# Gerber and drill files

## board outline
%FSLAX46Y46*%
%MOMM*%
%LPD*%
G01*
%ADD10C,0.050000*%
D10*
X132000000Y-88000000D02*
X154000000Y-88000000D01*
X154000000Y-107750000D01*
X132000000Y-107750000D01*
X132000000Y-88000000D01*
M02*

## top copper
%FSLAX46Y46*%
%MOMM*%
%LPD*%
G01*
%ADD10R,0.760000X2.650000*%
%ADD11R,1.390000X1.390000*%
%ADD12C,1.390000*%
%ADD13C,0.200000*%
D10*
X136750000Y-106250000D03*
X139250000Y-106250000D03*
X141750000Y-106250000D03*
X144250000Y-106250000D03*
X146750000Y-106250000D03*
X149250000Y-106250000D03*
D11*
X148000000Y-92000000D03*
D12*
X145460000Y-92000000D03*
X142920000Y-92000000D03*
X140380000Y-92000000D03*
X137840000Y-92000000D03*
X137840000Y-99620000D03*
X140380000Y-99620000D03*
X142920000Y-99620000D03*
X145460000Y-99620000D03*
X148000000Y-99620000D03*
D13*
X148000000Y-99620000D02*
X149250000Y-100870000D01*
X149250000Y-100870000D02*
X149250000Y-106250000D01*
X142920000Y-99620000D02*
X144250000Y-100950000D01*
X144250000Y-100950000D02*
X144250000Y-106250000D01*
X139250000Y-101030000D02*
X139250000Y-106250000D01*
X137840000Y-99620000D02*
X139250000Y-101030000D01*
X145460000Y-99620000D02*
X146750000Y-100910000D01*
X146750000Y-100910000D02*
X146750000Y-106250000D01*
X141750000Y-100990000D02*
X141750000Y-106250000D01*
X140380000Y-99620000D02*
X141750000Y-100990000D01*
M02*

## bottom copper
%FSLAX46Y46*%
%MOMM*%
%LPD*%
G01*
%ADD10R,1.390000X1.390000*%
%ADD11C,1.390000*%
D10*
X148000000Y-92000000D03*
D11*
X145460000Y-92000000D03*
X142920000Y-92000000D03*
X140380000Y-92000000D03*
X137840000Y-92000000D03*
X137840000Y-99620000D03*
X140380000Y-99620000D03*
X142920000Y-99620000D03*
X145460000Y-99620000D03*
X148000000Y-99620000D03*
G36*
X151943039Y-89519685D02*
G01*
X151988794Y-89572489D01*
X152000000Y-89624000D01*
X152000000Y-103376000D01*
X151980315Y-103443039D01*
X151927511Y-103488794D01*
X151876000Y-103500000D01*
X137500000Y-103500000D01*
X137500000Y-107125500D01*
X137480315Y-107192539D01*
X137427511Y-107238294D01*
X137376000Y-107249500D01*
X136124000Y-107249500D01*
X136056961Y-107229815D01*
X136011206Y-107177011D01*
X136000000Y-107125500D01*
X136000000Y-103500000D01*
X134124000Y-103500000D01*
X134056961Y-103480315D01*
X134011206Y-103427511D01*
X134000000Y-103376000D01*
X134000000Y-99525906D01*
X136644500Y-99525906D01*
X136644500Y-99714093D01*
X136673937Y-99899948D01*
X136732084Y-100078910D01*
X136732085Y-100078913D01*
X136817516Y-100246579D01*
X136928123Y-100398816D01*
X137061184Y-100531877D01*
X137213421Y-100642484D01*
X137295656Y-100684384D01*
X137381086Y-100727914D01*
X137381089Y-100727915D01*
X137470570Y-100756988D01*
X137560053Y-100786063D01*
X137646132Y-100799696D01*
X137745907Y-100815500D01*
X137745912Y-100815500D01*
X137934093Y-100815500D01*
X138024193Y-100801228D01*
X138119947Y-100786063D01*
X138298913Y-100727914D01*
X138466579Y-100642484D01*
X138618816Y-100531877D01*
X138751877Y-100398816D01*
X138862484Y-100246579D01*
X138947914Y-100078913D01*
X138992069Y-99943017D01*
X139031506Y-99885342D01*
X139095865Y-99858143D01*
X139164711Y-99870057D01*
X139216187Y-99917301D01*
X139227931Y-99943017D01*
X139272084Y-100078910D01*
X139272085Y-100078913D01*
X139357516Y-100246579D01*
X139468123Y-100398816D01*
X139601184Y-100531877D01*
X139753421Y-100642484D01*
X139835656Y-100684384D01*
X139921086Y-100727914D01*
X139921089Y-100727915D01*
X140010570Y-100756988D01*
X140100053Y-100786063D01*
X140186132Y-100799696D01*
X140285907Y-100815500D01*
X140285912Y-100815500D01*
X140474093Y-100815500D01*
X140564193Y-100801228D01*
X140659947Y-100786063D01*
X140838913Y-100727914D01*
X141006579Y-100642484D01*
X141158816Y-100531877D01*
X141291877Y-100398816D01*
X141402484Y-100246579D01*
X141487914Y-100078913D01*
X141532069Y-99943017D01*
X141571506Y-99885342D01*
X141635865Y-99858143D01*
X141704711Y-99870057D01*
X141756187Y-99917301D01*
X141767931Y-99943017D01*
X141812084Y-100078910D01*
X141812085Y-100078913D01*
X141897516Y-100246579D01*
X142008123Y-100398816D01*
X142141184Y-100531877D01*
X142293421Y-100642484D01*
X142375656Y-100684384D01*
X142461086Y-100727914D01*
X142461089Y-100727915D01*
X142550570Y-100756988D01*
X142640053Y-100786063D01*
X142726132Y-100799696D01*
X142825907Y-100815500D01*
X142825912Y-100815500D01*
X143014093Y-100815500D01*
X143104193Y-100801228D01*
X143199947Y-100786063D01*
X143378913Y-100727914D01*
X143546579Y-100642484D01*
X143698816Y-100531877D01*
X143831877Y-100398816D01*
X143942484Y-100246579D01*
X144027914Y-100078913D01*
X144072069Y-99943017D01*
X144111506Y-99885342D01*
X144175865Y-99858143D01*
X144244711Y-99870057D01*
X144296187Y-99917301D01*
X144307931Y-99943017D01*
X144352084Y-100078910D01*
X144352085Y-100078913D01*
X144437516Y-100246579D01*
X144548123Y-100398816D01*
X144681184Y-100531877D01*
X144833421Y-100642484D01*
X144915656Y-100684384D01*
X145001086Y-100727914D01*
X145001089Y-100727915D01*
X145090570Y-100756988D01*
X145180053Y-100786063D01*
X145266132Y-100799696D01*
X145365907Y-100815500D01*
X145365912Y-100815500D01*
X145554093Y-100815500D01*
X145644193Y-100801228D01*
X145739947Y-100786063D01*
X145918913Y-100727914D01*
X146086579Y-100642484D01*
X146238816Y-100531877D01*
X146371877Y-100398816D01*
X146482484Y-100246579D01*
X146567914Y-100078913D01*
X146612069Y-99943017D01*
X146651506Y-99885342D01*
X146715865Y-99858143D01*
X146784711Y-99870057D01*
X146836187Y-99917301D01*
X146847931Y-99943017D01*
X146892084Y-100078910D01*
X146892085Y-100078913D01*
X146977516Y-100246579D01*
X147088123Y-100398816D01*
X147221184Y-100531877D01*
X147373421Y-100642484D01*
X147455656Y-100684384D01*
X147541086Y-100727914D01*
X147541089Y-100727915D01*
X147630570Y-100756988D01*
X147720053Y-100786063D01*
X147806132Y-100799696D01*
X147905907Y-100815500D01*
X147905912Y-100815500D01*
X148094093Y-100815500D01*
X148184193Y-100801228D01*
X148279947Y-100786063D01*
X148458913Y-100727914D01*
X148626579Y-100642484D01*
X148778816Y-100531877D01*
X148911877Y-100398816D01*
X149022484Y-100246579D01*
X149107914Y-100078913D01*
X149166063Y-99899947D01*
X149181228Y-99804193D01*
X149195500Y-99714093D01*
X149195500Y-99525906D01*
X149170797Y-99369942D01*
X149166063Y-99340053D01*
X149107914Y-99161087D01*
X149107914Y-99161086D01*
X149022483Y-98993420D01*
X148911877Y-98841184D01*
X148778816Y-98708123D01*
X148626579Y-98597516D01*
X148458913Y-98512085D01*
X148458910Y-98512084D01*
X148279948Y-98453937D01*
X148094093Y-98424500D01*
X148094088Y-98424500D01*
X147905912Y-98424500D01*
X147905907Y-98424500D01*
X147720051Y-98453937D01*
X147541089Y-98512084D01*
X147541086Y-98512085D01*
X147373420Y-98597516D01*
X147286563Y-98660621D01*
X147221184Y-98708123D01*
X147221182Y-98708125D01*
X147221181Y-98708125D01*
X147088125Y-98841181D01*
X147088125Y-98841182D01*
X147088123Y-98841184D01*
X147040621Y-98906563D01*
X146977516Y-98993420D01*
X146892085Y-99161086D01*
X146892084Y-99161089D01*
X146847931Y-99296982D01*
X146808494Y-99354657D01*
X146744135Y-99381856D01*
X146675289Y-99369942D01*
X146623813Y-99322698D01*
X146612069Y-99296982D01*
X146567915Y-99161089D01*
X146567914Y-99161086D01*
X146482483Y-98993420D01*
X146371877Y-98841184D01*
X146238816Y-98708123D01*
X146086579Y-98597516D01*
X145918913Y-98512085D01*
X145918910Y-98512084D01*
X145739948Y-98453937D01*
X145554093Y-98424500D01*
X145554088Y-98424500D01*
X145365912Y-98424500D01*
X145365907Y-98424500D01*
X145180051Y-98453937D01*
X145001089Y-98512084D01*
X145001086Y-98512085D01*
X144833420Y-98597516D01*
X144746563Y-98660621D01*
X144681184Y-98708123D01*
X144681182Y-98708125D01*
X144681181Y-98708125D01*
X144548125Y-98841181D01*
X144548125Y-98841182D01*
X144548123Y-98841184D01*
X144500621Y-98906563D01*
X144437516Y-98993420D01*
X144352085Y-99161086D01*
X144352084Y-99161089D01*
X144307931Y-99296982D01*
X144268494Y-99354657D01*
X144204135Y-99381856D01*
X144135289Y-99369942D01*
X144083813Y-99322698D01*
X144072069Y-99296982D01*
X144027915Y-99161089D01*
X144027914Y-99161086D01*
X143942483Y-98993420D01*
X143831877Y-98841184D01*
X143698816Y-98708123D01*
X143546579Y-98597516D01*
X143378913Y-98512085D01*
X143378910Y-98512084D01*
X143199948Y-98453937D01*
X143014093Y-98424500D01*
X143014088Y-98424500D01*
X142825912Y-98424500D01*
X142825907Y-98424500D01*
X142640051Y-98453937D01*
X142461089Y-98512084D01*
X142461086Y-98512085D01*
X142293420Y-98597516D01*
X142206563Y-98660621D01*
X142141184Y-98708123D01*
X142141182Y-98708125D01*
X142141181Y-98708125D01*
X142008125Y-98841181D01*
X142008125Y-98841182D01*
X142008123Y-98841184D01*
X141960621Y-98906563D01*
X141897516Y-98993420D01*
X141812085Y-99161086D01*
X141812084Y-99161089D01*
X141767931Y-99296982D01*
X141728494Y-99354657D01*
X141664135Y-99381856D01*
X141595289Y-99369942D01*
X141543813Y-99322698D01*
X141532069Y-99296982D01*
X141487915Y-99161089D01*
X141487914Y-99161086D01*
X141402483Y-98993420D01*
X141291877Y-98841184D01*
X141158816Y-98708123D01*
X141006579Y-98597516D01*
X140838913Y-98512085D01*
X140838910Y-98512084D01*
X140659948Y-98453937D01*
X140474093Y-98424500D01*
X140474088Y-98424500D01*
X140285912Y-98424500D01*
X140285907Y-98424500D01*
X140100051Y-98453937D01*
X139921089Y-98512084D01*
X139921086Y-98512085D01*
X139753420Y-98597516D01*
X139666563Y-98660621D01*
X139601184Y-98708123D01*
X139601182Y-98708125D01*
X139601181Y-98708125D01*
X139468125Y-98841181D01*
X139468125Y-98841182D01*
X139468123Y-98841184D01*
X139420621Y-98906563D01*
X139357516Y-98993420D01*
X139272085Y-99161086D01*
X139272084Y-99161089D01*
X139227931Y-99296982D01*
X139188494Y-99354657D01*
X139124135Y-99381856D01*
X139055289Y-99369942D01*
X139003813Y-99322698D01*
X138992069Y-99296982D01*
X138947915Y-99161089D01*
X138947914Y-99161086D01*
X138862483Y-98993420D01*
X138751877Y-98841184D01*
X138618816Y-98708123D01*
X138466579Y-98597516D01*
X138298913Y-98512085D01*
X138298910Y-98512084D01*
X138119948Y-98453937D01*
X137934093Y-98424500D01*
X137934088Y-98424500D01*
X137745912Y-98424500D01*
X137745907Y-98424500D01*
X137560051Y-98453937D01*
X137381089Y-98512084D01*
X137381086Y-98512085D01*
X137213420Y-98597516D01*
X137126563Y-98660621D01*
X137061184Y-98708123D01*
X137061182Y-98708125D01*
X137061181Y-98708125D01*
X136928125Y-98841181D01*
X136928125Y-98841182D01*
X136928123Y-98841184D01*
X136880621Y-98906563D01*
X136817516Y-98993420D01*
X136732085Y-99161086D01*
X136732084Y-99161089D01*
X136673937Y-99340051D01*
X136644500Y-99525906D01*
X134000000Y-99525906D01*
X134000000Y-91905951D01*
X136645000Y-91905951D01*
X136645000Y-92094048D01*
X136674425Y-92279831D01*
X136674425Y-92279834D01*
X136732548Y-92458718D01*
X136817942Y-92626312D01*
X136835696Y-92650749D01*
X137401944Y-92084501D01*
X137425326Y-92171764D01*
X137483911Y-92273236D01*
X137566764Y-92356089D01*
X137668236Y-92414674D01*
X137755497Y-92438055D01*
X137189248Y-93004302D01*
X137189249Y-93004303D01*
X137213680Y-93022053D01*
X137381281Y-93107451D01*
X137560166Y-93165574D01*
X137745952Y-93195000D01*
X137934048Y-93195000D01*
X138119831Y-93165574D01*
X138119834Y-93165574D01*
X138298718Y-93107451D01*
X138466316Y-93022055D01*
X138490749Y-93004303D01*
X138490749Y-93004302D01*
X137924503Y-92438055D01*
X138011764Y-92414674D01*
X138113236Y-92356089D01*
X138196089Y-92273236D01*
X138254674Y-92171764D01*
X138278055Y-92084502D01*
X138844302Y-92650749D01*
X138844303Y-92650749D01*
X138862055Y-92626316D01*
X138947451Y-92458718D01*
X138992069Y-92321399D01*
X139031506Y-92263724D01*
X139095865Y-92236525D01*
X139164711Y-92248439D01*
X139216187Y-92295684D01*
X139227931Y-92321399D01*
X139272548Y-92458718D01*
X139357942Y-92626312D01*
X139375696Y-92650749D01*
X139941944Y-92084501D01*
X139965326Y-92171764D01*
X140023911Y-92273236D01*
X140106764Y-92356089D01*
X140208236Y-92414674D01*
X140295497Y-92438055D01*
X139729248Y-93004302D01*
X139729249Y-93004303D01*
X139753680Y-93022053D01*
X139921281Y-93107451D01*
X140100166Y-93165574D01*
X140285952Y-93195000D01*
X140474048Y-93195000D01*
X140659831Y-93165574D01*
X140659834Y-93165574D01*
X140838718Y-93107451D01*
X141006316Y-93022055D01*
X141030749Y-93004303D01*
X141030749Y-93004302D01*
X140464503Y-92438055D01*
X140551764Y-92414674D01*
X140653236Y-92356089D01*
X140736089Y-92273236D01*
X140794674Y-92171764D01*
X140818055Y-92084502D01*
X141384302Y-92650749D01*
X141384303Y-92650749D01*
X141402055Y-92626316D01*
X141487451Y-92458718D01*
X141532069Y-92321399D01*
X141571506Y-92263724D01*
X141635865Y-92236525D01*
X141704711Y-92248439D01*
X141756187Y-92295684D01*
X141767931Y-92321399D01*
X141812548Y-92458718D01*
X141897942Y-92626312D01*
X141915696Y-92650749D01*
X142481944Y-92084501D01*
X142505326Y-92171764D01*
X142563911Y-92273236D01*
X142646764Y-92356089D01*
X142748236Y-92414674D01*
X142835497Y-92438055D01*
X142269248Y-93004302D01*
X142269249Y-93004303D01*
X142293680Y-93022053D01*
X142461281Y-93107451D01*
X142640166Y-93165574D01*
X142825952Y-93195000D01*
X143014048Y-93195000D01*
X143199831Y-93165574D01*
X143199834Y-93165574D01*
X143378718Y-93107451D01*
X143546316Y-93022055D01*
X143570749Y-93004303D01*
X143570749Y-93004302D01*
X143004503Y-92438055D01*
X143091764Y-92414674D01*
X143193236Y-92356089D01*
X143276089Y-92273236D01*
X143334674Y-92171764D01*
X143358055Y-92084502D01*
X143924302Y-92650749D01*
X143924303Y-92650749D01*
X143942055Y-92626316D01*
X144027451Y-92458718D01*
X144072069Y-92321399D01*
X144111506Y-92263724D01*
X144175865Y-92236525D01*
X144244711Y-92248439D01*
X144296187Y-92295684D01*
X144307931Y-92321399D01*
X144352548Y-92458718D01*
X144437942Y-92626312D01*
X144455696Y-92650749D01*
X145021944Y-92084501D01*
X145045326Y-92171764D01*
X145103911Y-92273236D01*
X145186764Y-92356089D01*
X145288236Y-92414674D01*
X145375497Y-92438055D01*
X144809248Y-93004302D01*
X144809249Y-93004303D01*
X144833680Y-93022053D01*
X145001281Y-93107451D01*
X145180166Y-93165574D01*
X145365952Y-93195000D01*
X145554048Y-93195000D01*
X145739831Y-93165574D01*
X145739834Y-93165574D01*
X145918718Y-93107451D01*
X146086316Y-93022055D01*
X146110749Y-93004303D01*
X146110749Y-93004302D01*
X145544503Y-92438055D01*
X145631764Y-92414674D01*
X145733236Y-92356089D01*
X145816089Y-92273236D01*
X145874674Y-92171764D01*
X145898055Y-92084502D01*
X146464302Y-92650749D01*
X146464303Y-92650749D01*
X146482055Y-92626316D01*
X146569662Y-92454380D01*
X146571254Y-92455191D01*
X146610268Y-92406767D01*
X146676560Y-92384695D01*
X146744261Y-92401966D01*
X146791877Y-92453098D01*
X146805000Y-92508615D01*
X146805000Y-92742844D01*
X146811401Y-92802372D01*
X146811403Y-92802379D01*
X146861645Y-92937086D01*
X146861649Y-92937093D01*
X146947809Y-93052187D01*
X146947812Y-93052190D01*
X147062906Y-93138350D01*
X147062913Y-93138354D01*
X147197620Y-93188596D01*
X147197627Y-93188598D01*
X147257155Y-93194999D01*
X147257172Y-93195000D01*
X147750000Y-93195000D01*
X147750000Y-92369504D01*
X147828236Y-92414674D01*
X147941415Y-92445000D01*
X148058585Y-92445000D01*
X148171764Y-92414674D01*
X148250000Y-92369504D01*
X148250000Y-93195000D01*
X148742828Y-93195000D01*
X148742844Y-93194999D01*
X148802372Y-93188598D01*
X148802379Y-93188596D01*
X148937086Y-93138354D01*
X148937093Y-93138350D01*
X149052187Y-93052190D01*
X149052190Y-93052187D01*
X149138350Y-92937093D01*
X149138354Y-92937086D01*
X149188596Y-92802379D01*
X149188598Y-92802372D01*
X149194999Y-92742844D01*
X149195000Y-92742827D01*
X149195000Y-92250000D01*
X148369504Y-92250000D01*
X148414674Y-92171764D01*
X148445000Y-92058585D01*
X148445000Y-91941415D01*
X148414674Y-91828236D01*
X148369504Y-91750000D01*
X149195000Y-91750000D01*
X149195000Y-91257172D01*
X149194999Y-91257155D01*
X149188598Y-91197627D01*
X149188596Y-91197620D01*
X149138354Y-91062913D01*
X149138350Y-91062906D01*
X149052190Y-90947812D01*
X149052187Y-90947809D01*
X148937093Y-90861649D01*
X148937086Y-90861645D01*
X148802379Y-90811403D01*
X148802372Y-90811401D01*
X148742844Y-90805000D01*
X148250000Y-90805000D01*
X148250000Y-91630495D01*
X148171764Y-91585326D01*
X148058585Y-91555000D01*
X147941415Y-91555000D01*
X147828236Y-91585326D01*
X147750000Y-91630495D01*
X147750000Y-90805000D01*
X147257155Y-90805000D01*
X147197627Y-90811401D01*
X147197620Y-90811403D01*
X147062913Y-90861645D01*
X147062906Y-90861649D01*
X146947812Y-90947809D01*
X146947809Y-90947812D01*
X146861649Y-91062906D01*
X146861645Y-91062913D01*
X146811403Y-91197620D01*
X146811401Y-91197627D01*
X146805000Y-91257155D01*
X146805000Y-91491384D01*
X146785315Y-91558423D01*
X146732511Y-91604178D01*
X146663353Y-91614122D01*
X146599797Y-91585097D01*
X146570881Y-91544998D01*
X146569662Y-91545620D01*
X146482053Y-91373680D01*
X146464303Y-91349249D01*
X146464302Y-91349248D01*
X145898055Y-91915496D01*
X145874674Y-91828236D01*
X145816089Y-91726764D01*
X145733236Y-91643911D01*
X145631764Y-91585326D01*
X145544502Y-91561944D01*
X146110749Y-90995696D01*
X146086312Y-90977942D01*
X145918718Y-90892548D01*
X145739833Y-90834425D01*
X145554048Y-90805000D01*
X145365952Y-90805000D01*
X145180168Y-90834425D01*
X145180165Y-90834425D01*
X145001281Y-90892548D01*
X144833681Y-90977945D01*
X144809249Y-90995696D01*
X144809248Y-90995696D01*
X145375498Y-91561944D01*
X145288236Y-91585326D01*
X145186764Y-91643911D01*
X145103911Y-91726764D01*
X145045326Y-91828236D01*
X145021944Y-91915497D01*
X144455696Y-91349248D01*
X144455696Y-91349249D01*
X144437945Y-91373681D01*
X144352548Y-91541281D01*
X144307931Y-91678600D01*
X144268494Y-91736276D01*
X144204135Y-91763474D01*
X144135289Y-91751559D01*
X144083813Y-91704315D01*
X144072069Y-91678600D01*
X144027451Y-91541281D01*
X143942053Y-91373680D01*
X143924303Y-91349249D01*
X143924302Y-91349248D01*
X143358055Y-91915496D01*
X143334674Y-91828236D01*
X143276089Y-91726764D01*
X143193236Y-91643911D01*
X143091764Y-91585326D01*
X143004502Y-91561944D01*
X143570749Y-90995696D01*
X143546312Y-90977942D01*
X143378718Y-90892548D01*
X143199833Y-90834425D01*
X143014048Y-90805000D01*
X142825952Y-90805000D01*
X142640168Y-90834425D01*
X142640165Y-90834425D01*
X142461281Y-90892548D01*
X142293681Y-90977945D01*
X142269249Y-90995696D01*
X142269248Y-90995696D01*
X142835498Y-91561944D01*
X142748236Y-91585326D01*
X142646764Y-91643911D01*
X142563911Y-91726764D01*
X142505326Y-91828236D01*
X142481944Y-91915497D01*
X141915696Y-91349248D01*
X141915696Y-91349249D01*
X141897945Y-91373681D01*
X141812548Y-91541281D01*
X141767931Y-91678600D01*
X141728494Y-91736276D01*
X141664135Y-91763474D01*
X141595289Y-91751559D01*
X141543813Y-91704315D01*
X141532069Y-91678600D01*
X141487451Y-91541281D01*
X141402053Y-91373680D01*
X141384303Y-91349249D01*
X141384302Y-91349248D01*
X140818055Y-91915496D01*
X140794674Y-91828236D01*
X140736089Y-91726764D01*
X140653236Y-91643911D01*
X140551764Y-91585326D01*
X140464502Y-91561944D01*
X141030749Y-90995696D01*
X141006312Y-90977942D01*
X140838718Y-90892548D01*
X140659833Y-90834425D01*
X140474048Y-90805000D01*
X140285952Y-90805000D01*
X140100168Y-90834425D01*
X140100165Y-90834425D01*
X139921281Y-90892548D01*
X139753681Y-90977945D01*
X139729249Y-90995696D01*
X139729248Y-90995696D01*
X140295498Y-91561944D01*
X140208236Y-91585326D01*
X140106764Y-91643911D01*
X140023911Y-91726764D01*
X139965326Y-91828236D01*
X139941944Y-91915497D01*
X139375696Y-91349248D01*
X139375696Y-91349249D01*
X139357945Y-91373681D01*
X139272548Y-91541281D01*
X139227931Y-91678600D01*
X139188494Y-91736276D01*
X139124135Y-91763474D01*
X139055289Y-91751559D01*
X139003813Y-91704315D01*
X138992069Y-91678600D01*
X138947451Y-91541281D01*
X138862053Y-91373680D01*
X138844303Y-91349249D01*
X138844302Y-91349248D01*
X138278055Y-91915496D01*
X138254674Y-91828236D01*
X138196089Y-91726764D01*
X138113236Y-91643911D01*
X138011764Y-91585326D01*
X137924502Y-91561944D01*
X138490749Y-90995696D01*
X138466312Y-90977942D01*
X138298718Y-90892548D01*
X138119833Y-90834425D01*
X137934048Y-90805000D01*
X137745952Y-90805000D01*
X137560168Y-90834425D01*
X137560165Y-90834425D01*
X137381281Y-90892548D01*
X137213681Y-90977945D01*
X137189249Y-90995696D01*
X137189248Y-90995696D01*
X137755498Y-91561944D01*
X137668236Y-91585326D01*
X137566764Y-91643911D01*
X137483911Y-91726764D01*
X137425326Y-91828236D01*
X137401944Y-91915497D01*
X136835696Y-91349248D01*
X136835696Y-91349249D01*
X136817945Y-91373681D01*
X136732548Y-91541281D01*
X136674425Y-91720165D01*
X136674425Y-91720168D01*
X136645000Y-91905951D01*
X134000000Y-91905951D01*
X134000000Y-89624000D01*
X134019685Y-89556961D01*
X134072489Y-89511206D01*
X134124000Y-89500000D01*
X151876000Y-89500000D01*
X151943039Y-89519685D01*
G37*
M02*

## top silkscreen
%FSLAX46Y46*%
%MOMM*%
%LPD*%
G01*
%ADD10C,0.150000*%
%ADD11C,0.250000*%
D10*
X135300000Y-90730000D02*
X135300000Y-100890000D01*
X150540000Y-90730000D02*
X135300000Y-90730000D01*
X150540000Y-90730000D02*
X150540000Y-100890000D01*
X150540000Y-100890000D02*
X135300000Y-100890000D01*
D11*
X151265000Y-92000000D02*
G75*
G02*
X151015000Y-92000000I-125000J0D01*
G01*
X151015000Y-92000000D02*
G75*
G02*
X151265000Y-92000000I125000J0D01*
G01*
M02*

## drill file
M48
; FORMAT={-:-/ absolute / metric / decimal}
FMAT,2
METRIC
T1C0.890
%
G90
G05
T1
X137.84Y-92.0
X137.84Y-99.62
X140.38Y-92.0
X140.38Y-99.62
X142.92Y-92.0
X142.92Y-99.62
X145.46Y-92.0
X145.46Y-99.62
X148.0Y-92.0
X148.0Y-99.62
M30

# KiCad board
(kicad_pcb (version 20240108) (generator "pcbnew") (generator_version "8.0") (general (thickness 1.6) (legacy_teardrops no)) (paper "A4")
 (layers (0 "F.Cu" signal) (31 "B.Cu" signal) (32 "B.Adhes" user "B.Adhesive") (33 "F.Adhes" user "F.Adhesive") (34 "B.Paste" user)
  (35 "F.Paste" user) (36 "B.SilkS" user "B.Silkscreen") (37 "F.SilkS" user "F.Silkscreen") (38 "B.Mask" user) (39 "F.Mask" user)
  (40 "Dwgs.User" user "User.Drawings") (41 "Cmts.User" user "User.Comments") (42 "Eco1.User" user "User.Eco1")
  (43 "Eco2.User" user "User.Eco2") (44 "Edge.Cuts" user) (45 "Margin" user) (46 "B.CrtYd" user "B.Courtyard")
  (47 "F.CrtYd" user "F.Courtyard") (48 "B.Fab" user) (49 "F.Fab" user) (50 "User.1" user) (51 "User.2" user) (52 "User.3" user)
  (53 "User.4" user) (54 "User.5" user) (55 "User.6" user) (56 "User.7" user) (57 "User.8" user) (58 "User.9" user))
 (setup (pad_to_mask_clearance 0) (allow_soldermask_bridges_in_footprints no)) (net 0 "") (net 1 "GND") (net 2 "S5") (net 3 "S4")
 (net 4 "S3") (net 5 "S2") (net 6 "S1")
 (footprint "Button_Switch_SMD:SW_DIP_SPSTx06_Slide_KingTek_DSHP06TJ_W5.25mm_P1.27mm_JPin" (layer "F.Cu") (at 144.75 106.25)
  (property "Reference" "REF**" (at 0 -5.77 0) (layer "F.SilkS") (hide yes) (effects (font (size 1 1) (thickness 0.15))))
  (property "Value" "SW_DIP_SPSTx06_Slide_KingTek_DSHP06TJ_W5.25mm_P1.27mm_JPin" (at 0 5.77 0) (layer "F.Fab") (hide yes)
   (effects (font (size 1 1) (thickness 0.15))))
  (pad "1" smd rect (at -8 0 90) (size 2.65 0.76) (layers "F.Cu" "F.Paste" "F.Mask") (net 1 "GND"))
  (pad "2" smd rect (at -5.5 0 90) (size 2.65 0.76) (layers "F.Cu" "F.Paste" "F.Mask") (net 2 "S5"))
  (pad "3" smd rect (at -3 0 90) (size 2.65 0.76) (layers "F.Cu" "F.Paste" "F.Mask") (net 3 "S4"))
  (pad "4" smd rect (at -0.5 0 90) (size 2.65 0.76) (layers "F.Cu" "F.Paste" "F.Mask") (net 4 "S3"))
  (pad "5" smd rect (at 2 0 90) (size 2.65 0.76) (layers "F.Cu" "F.Paste" "F.Mask") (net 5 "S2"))
  (pad "6" smd rect (at 4.5 0 90) (size 2.65 0.76) (layers "F.Cu" "F.Paste" "F.Mask") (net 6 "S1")))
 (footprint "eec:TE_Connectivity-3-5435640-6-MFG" (layer "F.Cu") (at 142.92 95.81 180)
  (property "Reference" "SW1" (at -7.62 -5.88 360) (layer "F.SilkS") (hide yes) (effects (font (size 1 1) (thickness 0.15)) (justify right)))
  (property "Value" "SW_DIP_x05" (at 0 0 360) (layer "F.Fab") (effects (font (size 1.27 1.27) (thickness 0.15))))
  (fp_line (start 7.62 5.08) (end 7.62 -5.08) (stroke (width 0.15) (type solid)) (layer "F.SilkS"))
  (fp_line (start -7.62 5.08) (end 7.62 5.08) (stroke (width 0.15) (type solid)) (layer "F.SilkS"))
  (fp_line (start -7.62 5.08) (end -7.62 -5.08) (stroke (width 0.15) (type solid)) (layer "F.SilkS"))
  (fp_line (start -7.62 -5.08) (end 7.62 -5.08) (stroke (width 0.15) (type solid)) (layer "F.SilkS"))
  (fp_circle (center -8.22 3.81) (end -8.095 3.81) (stroke (width 0.25) (type solid)) (fill none) (layer "F.SilkS"))
  (pad "1" thru_hole rect (at -5.08 3.81 180) (size 1.39 1.39) (drill 0.89) (layers "*.Cu") (remove_unused_layers no) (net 1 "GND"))
  (pad "2" thru_hole circle (at -2.54 3.81 180) (size 1.39 1.39) (drill 0.89) (layers "*.Cu") (remove_unused_layers no) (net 1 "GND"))
  (pad "3" thru_hole circle (at 0 3.81 180) (size 1.39 1.39) (drill 0.89) (layers "*.Cu") (remove_unused_layers no) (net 1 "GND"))
  (pad "4" thru_hole circle (at 2.54 3.81 180) (size 1.39 1.39) (drill 0.89) (layers "*.Cu") (remove_unused_layers no) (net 1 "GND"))
  (pad "5" thru_hole circle (at 5.08 3.81 180) (size 1.39 1.39) (drill 0.89) (layers "*.Cu") (remove_unused_layers no) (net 1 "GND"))
  (pad "6" thru_hole circle (at 5.08 -3.81 180) (size 1.39 1.39) (drill 0.89) (layers "*.Cu") (remove_unused_layers no) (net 2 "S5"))
  (pad "7" thru_hole circle (at 2.54 -3.81 180) (size 1.39 1.39) (drill 0.89) (layers "*.Cu") (remove_unused_layers no) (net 3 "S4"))
  (pad "8" thru_hole circle (at 0 -3.81 180) (size 1.39 1.39) (drill 0.89) (layers "*.Cu") (remove_unused_layers no) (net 4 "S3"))
  (pad "9" thru_hole circle (at -2.54 -3.81 180) (size 1.39 1.39) (drill 0.89) (layers "*.Cu") (remove_unused_layers no) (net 5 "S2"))
  (pad "10" thru_hole circle (at -5.08 -3.81 180) (size 1.39 1.39) (drill 0.89) (layers "*.Cu") (remove_unused_layers no) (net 6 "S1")))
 (gr_rect (start 132 88) (end 154 107.75) (stroke (width 0.05) (type default)) (fill none) (layer "Edge.Cuts"))
 (segment (start 148 99.62) (end 149.25 100.87) (width 0.2) (layer "F.Cu") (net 6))
 (segment (start 149.25 100.87) (end 149.25 106.25) (width 0.2) (layer "F.Cu") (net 6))
 (segment (start 142.92 99.62) (end 144.25 100.95) (width 0.2) (layer "F.Cu") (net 4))
 (segment (start 144.25 100.95) (end 144.25 106.25) (width 0.2) (layer "F.Cu") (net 4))
 (segment (start 139.25 101.03) (end 139.25 106.25) (width 0.2) (layer "F.Cu") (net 2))
 (segment (start 137.84 99.62) (end 139.25 101.03) (width 0.2) (layer "F.Cu") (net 2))
 (segment (start 145.46 99.62) (end 146.75 100.91) (width 0.2) (layer "F.Cu") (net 5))
 (segment (start 146.75 100.91) (end 146.75 106.25) (width 0.2) (layer "F.Cu") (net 5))
 (segment (start 141.75 100.99) (end 141.75 106.25) (width 0.2) (layer "F.Cu") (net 3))
 (segment (start 140.38 99.62) (end 141.75 100.99) (width 0.2) (layer "F.Cu") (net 3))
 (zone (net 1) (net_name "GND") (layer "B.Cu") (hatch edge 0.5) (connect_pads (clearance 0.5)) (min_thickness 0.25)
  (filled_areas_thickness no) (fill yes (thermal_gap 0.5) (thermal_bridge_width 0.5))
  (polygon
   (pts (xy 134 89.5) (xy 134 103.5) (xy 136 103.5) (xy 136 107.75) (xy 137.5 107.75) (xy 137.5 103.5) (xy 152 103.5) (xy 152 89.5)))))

